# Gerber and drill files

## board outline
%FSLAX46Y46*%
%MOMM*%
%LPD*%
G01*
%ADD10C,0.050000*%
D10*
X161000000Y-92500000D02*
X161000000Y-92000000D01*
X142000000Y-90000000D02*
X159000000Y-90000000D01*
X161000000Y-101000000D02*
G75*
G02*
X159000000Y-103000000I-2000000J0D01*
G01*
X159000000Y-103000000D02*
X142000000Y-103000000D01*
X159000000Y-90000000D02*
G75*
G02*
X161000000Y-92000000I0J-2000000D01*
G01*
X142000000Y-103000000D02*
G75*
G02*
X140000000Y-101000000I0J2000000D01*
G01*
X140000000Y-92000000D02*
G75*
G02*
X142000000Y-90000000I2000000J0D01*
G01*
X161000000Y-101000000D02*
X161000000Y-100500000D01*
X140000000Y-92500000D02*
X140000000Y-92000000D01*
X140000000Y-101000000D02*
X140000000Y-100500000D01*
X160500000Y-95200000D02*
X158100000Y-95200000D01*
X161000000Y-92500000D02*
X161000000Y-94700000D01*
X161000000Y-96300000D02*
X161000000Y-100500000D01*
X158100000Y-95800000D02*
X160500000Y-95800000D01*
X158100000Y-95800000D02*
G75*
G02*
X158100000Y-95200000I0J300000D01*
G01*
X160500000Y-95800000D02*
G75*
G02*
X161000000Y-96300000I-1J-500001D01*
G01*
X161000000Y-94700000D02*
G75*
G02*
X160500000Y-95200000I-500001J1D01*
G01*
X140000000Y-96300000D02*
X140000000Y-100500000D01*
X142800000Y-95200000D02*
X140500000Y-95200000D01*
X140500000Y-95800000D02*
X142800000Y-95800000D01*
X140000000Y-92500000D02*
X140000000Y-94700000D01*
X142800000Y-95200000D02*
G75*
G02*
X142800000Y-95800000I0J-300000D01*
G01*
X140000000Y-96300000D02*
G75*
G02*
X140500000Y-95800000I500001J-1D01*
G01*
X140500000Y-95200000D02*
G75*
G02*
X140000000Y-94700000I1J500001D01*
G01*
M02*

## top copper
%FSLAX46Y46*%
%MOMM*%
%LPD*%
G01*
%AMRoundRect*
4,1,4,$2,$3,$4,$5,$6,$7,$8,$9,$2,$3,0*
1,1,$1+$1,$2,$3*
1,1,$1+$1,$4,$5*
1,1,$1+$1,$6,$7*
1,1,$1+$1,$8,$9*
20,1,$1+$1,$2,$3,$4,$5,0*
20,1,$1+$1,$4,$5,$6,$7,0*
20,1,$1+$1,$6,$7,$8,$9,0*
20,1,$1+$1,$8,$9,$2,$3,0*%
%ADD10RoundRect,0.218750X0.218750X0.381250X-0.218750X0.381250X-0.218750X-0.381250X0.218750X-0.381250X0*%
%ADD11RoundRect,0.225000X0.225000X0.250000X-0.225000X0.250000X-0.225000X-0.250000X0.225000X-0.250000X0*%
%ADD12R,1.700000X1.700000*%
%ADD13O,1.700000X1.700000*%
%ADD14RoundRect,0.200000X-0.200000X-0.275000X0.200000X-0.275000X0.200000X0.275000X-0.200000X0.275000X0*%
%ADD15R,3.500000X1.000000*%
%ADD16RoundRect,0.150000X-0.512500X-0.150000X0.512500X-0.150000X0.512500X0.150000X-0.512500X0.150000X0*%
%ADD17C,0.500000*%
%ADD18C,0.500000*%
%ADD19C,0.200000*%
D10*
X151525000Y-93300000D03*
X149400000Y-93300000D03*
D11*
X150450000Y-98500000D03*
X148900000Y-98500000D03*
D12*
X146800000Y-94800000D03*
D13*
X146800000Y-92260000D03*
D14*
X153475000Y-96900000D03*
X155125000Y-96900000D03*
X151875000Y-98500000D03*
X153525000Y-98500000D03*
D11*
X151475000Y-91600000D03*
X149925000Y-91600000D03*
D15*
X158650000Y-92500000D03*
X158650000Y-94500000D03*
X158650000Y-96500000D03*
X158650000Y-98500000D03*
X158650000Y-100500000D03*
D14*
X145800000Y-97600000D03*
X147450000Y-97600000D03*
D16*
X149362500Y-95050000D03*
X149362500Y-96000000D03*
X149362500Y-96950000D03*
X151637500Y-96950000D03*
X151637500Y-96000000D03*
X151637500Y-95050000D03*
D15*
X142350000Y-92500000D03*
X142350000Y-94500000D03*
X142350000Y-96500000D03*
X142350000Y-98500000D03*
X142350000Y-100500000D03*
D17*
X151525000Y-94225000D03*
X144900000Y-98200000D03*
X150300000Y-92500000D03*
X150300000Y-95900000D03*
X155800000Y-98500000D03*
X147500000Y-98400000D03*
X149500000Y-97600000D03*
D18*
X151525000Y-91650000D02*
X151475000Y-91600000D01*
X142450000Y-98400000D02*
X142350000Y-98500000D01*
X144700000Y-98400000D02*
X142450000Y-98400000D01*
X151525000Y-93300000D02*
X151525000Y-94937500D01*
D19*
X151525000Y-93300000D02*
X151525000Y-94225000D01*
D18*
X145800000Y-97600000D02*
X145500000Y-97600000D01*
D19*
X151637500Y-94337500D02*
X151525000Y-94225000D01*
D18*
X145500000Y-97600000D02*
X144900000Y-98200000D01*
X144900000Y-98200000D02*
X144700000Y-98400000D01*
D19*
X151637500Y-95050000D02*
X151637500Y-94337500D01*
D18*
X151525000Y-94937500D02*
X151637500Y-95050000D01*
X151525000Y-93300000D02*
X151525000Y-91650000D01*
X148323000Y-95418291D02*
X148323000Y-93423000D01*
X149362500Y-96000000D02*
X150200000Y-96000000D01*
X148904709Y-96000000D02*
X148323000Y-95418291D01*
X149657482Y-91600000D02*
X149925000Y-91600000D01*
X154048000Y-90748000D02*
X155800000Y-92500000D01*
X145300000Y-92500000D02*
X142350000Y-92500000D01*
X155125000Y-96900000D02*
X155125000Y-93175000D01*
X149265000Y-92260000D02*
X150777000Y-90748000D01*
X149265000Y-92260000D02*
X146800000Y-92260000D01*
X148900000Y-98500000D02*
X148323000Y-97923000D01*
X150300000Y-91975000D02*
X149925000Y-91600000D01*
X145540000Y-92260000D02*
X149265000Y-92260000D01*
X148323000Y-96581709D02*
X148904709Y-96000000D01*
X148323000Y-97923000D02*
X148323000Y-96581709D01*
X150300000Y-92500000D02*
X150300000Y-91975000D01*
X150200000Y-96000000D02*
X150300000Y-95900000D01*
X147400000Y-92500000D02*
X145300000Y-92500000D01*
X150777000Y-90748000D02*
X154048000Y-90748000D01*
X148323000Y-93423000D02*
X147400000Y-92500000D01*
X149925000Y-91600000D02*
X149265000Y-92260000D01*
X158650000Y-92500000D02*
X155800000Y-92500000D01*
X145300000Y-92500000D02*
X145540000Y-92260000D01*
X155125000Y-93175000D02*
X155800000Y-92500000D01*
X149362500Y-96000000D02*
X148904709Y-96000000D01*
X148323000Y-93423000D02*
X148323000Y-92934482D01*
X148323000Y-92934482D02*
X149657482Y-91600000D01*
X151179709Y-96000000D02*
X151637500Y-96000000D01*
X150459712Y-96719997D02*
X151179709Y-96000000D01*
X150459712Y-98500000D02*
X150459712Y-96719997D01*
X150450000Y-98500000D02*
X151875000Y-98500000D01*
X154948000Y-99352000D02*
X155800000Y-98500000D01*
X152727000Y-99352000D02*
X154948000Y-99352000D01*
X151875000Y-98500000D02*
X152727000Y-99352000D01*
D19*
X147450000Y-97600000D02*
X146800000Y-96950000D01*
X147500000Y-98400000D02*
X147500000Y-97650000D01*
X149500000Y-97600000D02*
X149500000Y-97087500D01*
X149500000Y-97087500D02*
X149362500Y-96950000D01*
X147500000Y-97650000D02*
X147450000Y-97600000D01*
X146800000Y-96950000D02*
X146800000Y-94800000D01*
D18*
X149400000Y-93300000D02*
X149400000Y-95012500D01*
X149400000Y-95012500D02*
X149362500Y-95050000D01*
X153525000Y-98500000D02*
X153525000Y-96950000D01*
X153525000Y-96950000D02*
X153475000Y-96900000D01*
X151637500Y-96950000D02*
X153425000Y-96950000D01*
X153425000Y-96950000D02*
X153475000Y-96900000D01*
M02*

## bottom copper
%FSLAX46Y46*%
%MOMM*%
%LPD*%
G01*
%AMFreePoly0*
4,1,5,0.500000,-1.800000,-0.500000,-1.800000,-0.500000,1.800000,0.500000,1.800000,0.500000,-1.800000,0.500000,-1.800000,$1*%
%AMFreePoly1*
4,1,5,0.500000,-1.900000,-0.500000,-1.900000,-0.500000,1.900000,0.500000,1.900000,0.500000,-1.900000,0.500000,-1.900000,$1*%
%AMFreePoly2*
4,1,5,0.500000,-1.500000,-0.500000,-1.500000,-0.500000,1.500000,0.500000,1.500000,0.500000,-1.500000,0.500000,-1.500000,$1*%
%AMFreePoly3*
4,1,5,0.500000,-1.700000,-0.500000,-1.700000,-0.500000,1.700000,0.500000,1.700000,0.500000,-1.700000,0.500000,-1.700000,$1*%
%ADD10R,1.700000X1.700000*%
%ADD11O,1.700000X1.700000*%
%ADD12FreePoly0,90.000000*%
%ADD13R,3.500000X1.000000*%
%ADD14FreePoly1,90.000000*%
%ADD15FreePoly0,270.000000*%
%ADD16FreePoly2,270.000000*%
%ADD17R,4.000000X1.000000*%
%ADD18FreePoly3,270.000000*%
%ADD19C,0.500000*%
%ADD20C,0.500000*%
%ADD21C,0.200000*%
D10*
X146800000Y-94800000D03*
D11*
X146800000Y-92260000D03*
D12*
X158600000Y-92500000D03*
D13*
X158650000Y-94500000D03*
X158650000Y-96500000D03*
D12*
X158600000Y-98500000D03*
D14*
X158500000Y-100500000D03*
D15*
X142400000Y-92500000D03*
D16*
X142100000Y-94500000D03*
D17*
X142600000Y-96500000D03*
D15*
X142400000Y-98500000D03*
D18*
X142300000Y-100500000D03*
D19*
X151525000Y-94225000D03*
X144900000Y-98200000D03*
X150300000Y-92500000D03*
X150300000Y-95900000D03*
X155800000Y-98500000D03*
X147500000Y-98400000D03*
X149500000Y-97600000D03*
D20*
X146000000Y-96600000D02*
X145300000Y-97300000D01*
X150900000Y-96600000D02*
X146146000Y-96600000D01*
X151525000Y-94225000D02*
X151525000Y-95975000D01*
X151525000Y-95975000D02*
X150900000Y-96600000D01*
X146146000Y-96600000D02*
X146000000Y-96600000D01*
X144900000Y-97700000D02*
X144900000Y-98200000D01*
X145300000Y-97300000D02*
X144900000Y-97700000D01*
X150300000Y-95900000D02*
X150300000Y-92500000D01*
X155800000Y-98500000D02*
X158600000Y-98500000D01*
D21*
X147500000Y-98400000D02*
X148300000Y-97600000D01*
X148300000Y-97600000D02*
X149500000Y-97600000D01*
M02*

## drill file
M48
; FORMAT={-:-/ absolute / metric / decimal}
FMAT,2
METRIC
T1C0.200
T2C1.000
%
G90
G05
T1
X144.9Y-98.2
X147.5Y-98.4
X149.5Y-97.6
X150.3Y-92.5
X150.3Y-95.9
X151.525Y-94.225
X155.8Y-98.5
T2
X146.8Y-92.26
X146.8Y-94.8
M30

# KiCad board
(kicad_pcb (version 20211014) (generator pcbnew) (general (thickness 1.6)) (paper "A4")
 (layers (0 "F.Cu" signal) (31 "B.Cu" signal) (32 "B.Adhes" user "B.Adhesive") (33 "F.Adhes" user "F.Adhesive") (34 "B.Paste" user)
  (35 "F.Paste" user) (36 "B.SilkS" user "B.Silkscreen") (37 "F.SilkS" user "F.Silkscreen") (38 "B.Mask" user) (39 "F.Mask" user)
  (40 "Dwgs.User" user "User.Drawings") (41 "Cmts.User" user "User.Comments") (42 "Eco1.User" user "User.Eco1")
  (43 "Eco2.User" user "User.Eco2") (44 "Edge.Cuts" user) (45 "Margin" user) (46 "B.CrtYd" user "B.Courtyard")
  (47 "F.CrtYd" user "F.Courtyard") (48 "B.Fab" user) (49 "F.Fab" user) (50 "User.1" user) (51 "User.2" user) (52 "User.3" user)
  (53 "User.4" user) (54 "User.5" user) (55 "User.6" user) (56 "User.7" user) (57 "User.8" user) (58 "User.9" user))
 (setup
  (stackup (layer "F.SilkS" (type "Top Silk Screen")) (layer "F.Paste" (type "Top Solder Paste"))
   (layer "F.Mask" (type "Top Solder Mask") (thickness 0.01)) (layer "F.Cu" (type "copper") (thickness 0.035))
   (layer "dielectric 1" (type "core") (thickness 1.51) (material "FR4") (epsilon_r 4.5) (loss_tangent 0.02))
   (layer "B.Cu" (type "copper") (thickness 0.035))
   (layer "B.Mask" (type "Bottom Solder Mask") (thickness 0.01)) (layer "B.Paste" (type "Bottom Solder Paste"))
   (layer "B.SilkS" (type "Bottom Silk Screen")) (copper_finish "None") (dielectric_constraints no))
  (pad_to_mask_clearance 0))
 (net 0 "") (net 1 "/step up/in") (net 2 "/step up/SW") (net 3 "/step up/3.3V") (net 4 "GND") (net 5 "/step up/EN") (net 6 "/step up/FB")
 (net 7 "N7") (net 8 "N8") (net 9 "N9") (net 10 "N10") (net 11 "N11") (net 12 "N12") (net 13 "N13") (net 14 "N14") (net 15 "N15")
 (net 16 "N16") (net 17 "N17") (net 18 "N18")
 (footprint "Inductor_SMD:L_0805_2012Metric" (layer "F.Cu") (at 150.4625 93.3 180)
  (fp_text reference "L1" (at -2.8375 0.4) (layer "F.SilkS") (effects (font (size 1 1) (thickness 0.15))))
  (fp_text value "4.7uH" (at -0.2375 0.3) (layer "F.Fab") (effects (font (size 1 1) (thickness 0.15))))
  (pad "1" smd roundrect (at -1.0625 0 180) (size 0.875 1.2) (layers "F.Cu" "F.Paste" "F.Mask") (roundrect_rratio 0.25)
   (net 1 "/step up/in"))
  (pad "2" smd roundrect (at 1.0625 0 180) (size 0.875 1.2) (layers "F.Cu" "F.Paste" "F.Mask") (roundrect_rratio 0.25) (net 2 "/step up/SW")))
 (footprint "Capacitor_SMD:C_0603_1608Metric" (layer "F.Cu") (at 149.675 98.5 180)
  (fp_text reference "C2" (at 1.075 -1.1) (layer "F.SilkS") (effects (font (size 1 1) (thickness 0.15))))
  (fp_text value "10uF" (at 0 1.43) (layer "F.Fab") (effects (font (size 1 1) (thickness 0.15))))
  (pad "1" smd roundrect (at -0.775 0 180) (size 0.9 0.95) (layers "F.Cu" "F.Paste" "F.Mask") (roundrect_rratio 0.25)
   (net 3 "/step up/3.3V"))
  (pad "2" smd roundrect (at 0.775 0 180) (size 0.9 0.95) (layers "F.Cu" "F.Paste" "F.Mask") (roundrect_rratio 0.25) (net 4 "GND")))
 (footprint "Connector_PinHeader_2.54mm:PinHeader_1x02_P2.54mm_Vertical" (layer "F.Cu") (at 146.8 94.8 180)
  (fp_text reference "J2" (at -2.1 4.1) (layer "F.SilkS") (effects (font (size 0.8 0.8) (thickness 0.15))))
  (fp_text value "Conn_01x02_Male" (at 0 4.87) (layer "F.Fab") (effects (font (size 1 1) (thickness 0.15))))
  (pad "1" thru_hole rect (at 0 0 180) (size 1.7 1.7) (drill 1) (layers *.Cu *.Mask) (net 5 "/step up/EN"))
  (pad "2" thru_hole oval (at 0 2.54 180) (size 1.7 1.7) (drill 1) (layers *.Cu *.Mask) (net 4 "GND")))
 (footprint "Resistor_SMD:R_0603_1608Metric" (layer "F.Cu") (at 154.3 96.9)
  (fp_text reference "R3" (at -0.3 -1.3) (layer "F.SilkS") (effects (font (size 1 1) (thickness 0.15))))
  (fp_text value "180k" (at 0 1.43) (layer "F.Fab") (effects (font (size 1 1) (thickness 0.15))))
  (pad "1" smd roundrect (at -0.825 0) (size 0.8 0.95) (layers "F.Cu" "F.Paste" "F.Mask") (roundrect_rratio 0.25) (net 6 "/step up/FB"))
  (pad "2" smd roundrect (at 0.825 0) (size 0.8 0.95) (layers "F.Cu" "F.Paste" "F.Mask") (roundrect_rratio 0.25) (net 4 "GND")))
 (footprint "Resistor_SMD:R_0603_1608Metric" (layer "F.Cu") (at 152.7 98.5)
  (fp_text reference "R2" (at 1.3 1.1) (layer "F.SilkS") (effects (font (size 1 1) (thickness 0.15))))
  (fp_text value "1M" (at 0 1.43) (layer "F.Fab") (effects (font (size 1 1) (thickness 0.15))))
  (pad "1" smd roundrect (at -0.825 0) (size 0.8 0.95) (layers "F.Cu" "F.Paste" "F.Mask") (roundrect_rratio 0.25) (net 3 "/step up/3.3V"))
  (pad "2" smd roundrect (at 0.825 0) (size 0.8 0.95) (layers "F.Cu" "F.Paste" "F.Mask") (roundrect_rratio 0.25) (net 6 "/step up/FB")))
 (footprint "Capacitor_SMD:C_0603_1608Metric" (layer "F.Cu") (at 150.7 91.6 180)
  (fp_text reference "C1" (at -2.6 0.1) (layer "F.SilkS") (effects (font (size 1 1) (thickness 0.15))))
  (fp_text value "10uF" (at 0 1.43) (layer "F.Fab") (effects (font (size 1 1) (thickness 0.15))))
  (pad "1" smd roundrect (at -0.775 0 180) (size 0.9 0.95) (layers "F.Cu" "F.Paste" "F.Mask") (roundrect_rratio 0.25) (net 1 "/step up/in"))
  (pad "2" smd roundrect (at 0.775 0 180) (size 0.9 0.95) (layers "F.Cu" "F.Paste" "F.Mask") (roundrect_rratio 0.25) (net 4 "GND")))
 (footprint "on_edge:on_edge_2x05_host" (layer "F.Cu") (at 161 96.5 -90)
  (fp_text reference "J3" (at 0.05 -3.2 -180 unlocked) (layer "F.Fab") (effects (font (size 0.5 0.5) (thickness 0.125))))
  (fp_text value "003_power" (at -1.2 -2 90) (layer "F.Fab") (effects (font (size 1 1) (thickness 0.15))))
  (fp_line (start -1.3 0.5) (end -1.3 2.9) (layer "Edge.Cuts") (width 0.05))
  (fp_line (start -4 0) (end -1.8 0) (layer "Edge.Cuts") (width 0.05))
  (fp_line (start -0.2 0) (end 4 0) (layer "Edge.Cuts") (width 0.05))
  (fp_line (start -0.7 2.9) (end -0.7 0.5) (layer "Edge.Cuts") (width 0.05))
  (fp_arc (start -0.7 2.9) (mid -1 3.2) (end -1.3 2.9) (layer "Edge.Cuts") (width 0.05))
  (fp_arc (start -0.7 0.5) (mid -0.553553 0.146447) (end -0.2 0) (layer "Edge.Cuts") (width 0.05))
  (fp_arc (start -1.8 0) (mid -1.446447 0.146447) (end -1.3 0.5) (layer "Edge.Cuts") (width 0.05))
  (pad "1" smd rect (at -4 2.35 270) (size 1 3.5) (layers "F.Cu" "F.Mask") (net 4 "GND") (zone_connect 0))
  (pad "2" smd rect (at -2 2.35 270) (size 1 3.5) (layers "F.Cu" "F.Mask") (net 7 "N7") (zone_connect 0))
  (pad "3" smd rect (at 0 2.35 270) (size 1 3.5) (layers "F.Cu" "F.Mask") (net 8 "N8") (zone_connect 0))
  (pad "4" smd rect (at 2 2.35 270) (size 1 3.5) (layers "F.Cu" "F.Mask") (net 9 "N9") (zone_connect 0))
  (pad "5" smd rect (at 4 2.35 270) (size 1 3.5) (layers "F.Cu" "F.Mask") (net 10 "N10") (zone_connect 0))
  (pad "6" smd custom (at -4 2.4 90) (size 1 3.6) (layers "B.Cu" "B.Mask") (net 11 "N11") (zone_connect 0)
   (options (clearance outline) (anchor rect)) (primitives))
  (pad "7" smd rect (at -2 2.35 90) (size 1 3.5) (layers "B.Cu" "B.Mask") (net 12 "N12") (zone_connect 0))
  (pad "8" smd rect (at 0 2.35 90) (size 1 3.5) (layers "B.Cu" "B.Mask") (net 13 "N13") (zone_connect 0))
  (pad "9" smd custom (at 2 2.4 90) (size 1 3.6) (layers "B.Cu" "B.Mask") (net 3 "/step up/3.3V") (zone_connect 0)
   (options (clearance outline) (anchor rect)) (primitives))
  (pad "10" smd custom (at 4 2.5 90) (size 1 3.8) (layers "B.Cu" "B.Mask") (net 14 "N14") (zone_connect 0)
   (options (clearance outline) (anchor rect)) (primitives)))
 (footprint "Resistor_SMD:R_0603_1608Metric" (layer "F.Cu") (at 146.625 97.6)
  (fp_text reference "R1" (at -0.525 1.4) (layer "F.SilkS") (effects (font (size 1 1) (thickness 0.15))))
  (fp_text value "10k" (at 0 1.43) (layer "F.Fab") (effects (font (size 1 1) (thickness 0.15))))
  (pad "1" smd roundrect (at -0.825 0) (size 0.8 0.95) (layers "F.Cu" "F.Paste" "F.Mask") (roundrect_rratio 0.25) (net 1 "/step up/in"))
  (pad "2" smd roundrect (at 0.825 0) (size 0.8 0.95) (layers "F.Cu" "F.Paste" "F.Mask") (roundrect_rratio 0.25) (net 5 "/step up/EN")))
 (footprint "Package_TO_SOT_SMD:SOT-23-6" (layer "F.Cu") (at 150.5 96)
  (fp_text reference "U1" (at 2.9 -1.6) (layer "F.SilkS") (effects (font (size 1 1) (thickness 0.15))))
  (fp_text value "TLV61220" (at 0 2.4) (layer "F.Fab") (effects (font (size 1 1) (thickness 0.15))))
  (pad "1" smd roundrect (at -1.1375 -0.95) (size 1.325 0.6) (layers "F.Cu" "F.Paste" "F.Mask") (roundrect_rratio 0.25)
   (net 2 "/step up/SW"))
  (pad "2" smd roundrect (at -1.1375 0) (size 1.325 0.6) (layers "F.Cu" "F.Paste" "F.Mask") (roundrect_rratio 0.25) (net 4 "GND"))
  (pad "3" smd roundrect (at -1.1375 0.95) (size 1.325 0.6) (layers "F.Cu" "F.Paste" "F.Mask") (roundrect_rratio 0.25) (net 5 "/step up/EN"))
  (pad "4" smd roundrect (at 1.1375 0.95) (size 1.325 0.6) (layers "F.Cu" "F.Paste" "F.Mask") (roundrect_rratio 0.25) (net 6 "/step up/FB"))
  (pad "5" smd roundrect (at 1.1375 0) (size 1.325 0.6) (layers "F.Cu" "F.Paste" "F.Mask") (roundrect_rratio 0.25) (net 3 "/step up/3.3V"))
  (pad "6" smd roundrect (at 1.1375 -0.95) (size 1.325 0.6) (layers "F.Cu" "F.Paste" "F.Mask") (roundrect_rratio 0.25) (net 1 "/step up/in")))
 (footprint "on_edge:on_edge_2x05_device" (layer "F.Cu") (at 140 96.5 -90)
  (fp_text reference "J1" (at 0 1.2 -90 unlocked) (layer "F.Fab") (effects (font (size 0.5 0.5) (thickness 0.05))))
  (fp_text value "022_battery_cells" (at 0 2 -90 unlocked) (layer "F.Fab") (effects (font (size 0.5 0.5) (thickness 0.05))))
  (fp_line (start -0.2 0) (end 4 0) (layer "Edge.Cuts") (width 0.05))
  (fp_line (start -1.3 -2.8) (end -1.3 -0.5) (layer "Edge.Cuts") (width 0.05))
  (fp_line (start -0.7 -0.5) (end -0.7 -2.8) (layer "Edge.Cuts") (width 0.05))
  (fp_line (start -4 0) (end -1.8 0) (layer "Edge.Cuts") (width 0.05))
  (fp_arc (start -1.3 -2.8) (mid -1 -3.1) (end -0.7 -2.8) (layer "Edge.Cuts") (width 0.05))
  (fp_arc (start -0.2 0) (mid -0.553553 -0.146447) (end -0.7 -0.5) (layer "Edge.Cuts") (width 0.05))
  (fp_arc (start -1.3 -0.5) (mid -1.446447 -0.146447) (end -1.8 0) (layer "Edge.Cuts") (width 0.05))
  (pad "1" smd rect (at -4 -2.35 90) (size 1 3.5) (layers "F.Cu" "F.Mask") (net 4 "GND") (zone_connect 0))
  (pad "2" smd rect (at -2 -2.35 270) (size 1 3.5) (layers "F.Cu" "F.Mask") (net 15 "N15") (zone_connect 0))
  (pad "3" smd rect (at 0 -2.35 270) (size 1 3.5) (layers "F.Cu" "F.Mask") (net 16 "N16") (zone_connect 0))
  (pad "4" smd rect (at 2 -2.35 90) (size 1 3.5) (layers "F.Cu" "F.Mask") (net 1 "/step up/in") (zone_connect 0))
  (pad "5" smd rect (at 4 -2.35 90) (size 1 3.5) (layers "F.Cu" "F.Mask") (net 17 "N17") (zone_connect 0))
  (pad "6" smd custom (at -4 -2.4 270) (size 1 3.6) (layers "B.Cu" "B.Mask") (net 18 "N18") (zone_connect 0)
   (options (clearance outline) (anchor rect)) (primitives))
  (pad "7" smd custom (at -2 -2.1 270) (size 1 3) (layers "B.Cu" "B.Mask") (zone_connect 0) (options (clearance outline) (anchor rect))
   (primitives))
  (pad "8" smd rect (at 0 -2.6 270) (size 1 4) (layers "B.Cu" "B.Mask") (zone_connect 0))
  (pad "9" smd custom (at 2 -2.4 270) (size 1 3.6) (layers "B.Cu" "B.Mask") (zone_connect 0) (options (clearance outline) (anchor rect))
   (primitives))
  (pad "10" smd custom (at 4 -2.3 270) (size 1 3.4) (layers "B.Cu" "B.Mask") (zone_connect 0) (options (clearance outline) (anchor rect))
   (primitives))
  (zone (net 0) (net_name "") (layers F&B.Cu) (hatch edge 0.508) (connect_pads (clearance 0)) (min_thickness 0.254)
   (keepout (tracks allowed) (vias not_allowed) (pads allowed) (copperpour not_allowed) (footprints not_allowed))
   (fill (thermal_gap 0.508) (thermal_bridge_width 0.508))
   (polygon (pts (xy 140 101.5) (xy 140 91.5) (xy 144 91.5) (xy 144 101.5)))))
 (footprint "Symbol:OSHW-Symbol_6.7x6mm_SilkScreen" (layer "B.Cu") (at 150 99 180)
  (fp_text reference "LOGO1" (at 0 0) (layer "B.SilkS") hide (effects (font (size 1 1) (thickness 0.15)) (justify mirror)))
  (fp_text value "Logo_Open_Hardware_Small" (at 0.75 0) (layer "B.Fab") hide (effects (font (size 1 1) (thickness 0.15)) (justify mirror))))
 (gr_line (start 161 92.5) (end 161 92) (layer "Edge.Cuts") (width 0.05))
 (gr_line (start 142 90) (end 159 90) (layer "Edge.Cuts") (width 0.05))
 (gr_arc (start 161 101) (mid 160.414214 102.414214) (end 159 103) (layer "Edge.Cuts") (width 0.05))
 (gr_line (start 159 103) (end 142 103) (layer "Edge.Cuts") (width 0.05))
 (gr_arc (start 159 90) (mid 160.414214 90.585786) (end 161 92) (layer "Edge.Cuts") (width 0.05))
 (gr_arc (start 142 103) (mid 140.585786 102.414214) (end 140 101) (layer "Edge.Cuts") (width 0.05))
 (gr_arc (start 140 92) (mid 140.585786 90.585786) (end 142 90) (layer "Edge.Cuts") (width 0.05))
 (gr_line (start 161 101) (end 161 100.5) (layer "Edge.Cuts") (width 0.05))
 (gr_line (start 140 92.5) (end 140 92) (layer "Edge.Cuts") (width 0.05))
 (gr_line (start 140 101) (end 140 100.5) (layer "Edge.Cuts") (width 0.05))
 (segment (start 151.525 91.65) (end 151.475 91.6) (width 0.5) (layer "F.Cu") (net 1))
 (segment (start 142.45 98.4) (end 142.35 98.5) (width 0.5) (layer "F.Cu") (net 1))
 (segment (start 144.7 98.4) (end 142.45 98.4) (width 0.5) (layer "F.Cu") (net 1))
 (segment (start 151.525 93.3) (end 151.525 94.9375) (width 0.5) (layer "F.Cu") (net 1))
 (segment (start 151.525 93.3) (end 151.525 94.225) (width 0.2) (layer "F.Cu") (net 1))
 (segment (start 145.8 97.6) (end 145.5 97.6) (width 0.5) (layer "F.Cu") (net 1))
 (segment (start 151.6375 94.3375) (end 151.525 94.225) (width 0.2) (layer "F.Cu") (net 1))
 (segment (start 145.5 97.6) (end 144.9 98.2) (width 0.5) (layer "F.Cu") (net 1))
 (segment (start 144.9 98.2) (end 144.7 98.4) (width 0.5) (layer "F.Cu") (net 1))
 (segment (start 151.6375 95.05) (end 151.6375 94.3375) (width 0.2) (layer "F.Cu") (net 1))
 (segment (start 151.525 94.9375) (end 151.6375 95.05) (width 0.5) (layer "F.Cu") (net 1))
 (segment (start 151.525 93.3) (end 151.525 91.65) (width 0.5) (layer "F.Cu") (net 1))
 (via (at 151.525 94.225) (size 0.5) (drill 0.2) (layers "F.Cu" "B.Cu") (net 1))
 (via (at 144.9 98.2) (size 0.5) (drill 0.2) (layers "F.Cu" "B.Cu") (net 1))
 (segment (start 146 96.6) (end 145.3 97.3) (width 0.5) (layer "B.Cu") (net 1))
 (segment (start 150.9 96.6) (end 146.146 96.6) (width 0.5) (layer "B.Cu") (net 1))
 (segment (start 151.525 94.225) (end 151.525 95.975) (width 0.5) (layer "B.Cu") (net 1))
 (segment (start 151.525 95.975) (end 150.9 96.6) (width 0.5) (layer "B.Cu") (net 1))
 (segment (start 146.146 96.6) (end 146 96.6) (width 0.5) (layer "B.Cu") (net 1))
 (segment (start 144.9 97.7) (end 144.9 98.2) (width 0.5) (layer "B.Cu") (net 1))
 (segment (start 145.3 97.3) (end 144.9 97.7) (width 0.5) (layer "B.Cu") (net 1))
 (segment (start 148.323 95.418291) (end 148.323 93.423) (width 0.5) (layer "F.Cu") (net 4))
 (segment (start 149.3625 96) (end 150.2 96) (width 0.5) (layer "F.Cu") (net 4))
 (segment (start 148.904709 96) (end 148.323 95.418291) (width 0.5) (layer "F.Cu") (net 4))
 (segment (start 149.657482 91.6) (end 149.925 91.6) (width 0.5) (layer "F.Cu") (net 4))
 (segment (start 154.048 90.748) (end 155.8 92.5) (width 0.5) (layer "F.Cu") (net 4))
 (segment (start 145.3 92.5) (end 142.35 92.5) (width 0.5) (layer "F.Cu") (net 4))
 (segment (start 155.125 96.9) (end 155.125 93.175) (width 0.5) (layer "F.Cu") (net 4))
 (segment (start 149.265 92.26) (end 150.777 90.748) (width 0.5) (layer "F.Cu") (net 4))
 (segment (start 149.265 92.26) (end 146.8 92.26) (width 0.5) (layer "F.Cu") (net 4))
 (segment (start 148.9 98.5) (end 148.323 97.923) (width 0.5) (layer "F.Cu") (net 4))
 (segment (start 150.3 91.975) (end 149.925 91.6) (width 0.5) (layer "F.Cu") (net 4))
 (segment (start 145.54 92.26) (end 149.265 92.26) (width 0.5) (layer "F.Cu") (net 4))
 (segment (start 148.323 96.581709) (end 148.904709 96) (width 0.5) (layer "F.Cu") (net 4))
 (segment (start 148.323 97.923) (end 148.323 96.581709) (width 0.5) (layer "F.Cu") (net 4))
 (segment (start 150.3 92.5) (end 150.3 91.975) (width 0.5) (layer "F.Cu") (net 4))
 (segment (start 150.2 96) (end 150.3 95.9) (width 0.5) (layer "F.Cu") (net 4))
 (segment (start 147.4 92.5) (end 145.3 92.5) (width 0.5) (layer "F.Cu") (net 4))
 (segment (start 150.777 90.748) (end 154.048 90.748) (width 0.5) (layer "F.Cu") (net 4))
 (segment (start 148.323 93.423) (end 147.4 92.5) (width 0.5) (layer "F.Cu") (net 4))
 (segment (start 149.925 91.6) (end 149.265 92.26) (width 0.5) (layer "F.Cu") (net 4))
 (segment (start 158.65 92.5) (end 155.8 92.5) (width 0.5) (layer "F.Cu") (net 4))
 (segment (start 145.3 92.5) (end 145.54 92.26) (width 0.5) (layer "F.Cu") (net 4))
 (segment (start 155.125 93.175) (end 155.8 92.5) (width 0.5) (layer "F.Cu") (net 4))
 (segment (start 149.3625 96) (end 148.904709 96) (width 0.5) (layer "F.Cu") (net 4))
 (segment (start 148.323 93.423) (end 148.323 92.934482) (width 0.5) (layer "F.Cu") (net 4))
 (segment (start 148.323 92.934482) (end 149.657482 91.6) (width 0.5) (layer "F.Cu") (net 4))
 (via (at 150.3 92.5) (size 0.5) (drill 0.2) (layers "F.Cu" "B.Cu") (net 4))
 (via (at 150.3 95.9) (size 0.5) (drill 0.2) (layers "F.Cu" "B.Cu") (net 4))
 (segment (start 150.3 95.9) (end 150.3 92.5) (width 0.5) (layer "B.Cu") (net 4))
 (segment (start 151.179709 96) (end 151.6375 96) (width 0.5) (layer "F.Cu") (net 3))
 (segment (start 150.459712 96.719997) (end 151.179709 96) (width 0.5) (layer "F.Cu") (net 3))
 (segment (start 150.459712 98.5) (end 150.459712 96.719997) (width 0.5) (layer "F.Cu") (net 3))
 (segment (start 150.45 98.5) (end 151.875 98.5) (width 0.5) (layer "F.Cu") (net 3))
 (segment (start 154.948 99.352) (end 155.8 98.5) (width 0.5) (layer "F.Cu") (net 3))
 (segment (start 152.727 99.352) (end 154.948 99.352) (width 0.5) (layer "F.Cu") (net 3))
 (segment (start 151.875 98.5) (end 152.727 99.352) (width 0.5) (layer "F.Cu") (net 3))
 (via (at 155.8 98.5) (size 0.5) (drill 0.2) (layers "F.Cu" "B.Cu") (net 3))
 (segment (start 155.8 98.5) (end 158.6 98.5) (width 0.5) (layer "B.Cu") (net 3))
 (segment (start 147.45 97.6) (end 146.8 96.95) (width 0.2) (layer "F.Cu") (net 5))
 (segment (start 147.5 98.4) (end 147.5 97.65) (width 0.2) (layer "F.Cu") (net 5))
 (segment (start 149.5 97.6) (end 149.5 97.0875) (width 0.2) (layer "F.Cu") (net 5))
 (segment (start 149.5 97.0875) (end 149.3625 96.95) (width 0.2) (layer "F.Cu") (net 5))
 (segment (start 147.5 97.65) (end 147.45 97.6) (width 0.2) (layer "F.Cu") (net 5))
 (segment (start 146.8 96.95) (end 146.8 94.8) (width 0.2) (layer "F.Cu") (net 5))
 (via (at 147.5 98.4) (size 0.5) (drill 0.2) (layers "F.Cu" "B.Cu") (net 5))
 (via (at 149.5 97.6) (size 0.5) (drill 0.2) (layers "F.Cu" "B.Cu") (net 5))
 (segment (start 147.5 98.4) (end 148.3 97.6) (width 0.2) (layer "B.Cu") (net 5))
 (segment (start 148.3 97.6) (end 149.5 97.6) (width 0.2) (layer "B.Cu") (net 5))
 (segment (start 149.4 93.3) (end 149.4 95.0125) (width 0.5) (layer "F.Cu") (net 2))
 (segment (start 149.4 95.0125) (end 149.3625 95.05) (width 0.5) (layer "F.Cu") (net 2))
 (segment (start 153.525 98.5) (end 153.525 96.95) (width 0.5) (layer "F.Cu") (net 6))
 (segment (start 153.525 96.95) (end 153.475 96.9) (width 0.5) (layer "F.Cu") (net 6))
 (segment (start 151.6375 96.95) (end 153.425 96.95) (width 0.5) (layer "F.Cu") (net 6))
 (segment (start 153.425 96.95) (end 153.475 96.9) (width 0.5) (layer "F.Cu") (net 6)))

